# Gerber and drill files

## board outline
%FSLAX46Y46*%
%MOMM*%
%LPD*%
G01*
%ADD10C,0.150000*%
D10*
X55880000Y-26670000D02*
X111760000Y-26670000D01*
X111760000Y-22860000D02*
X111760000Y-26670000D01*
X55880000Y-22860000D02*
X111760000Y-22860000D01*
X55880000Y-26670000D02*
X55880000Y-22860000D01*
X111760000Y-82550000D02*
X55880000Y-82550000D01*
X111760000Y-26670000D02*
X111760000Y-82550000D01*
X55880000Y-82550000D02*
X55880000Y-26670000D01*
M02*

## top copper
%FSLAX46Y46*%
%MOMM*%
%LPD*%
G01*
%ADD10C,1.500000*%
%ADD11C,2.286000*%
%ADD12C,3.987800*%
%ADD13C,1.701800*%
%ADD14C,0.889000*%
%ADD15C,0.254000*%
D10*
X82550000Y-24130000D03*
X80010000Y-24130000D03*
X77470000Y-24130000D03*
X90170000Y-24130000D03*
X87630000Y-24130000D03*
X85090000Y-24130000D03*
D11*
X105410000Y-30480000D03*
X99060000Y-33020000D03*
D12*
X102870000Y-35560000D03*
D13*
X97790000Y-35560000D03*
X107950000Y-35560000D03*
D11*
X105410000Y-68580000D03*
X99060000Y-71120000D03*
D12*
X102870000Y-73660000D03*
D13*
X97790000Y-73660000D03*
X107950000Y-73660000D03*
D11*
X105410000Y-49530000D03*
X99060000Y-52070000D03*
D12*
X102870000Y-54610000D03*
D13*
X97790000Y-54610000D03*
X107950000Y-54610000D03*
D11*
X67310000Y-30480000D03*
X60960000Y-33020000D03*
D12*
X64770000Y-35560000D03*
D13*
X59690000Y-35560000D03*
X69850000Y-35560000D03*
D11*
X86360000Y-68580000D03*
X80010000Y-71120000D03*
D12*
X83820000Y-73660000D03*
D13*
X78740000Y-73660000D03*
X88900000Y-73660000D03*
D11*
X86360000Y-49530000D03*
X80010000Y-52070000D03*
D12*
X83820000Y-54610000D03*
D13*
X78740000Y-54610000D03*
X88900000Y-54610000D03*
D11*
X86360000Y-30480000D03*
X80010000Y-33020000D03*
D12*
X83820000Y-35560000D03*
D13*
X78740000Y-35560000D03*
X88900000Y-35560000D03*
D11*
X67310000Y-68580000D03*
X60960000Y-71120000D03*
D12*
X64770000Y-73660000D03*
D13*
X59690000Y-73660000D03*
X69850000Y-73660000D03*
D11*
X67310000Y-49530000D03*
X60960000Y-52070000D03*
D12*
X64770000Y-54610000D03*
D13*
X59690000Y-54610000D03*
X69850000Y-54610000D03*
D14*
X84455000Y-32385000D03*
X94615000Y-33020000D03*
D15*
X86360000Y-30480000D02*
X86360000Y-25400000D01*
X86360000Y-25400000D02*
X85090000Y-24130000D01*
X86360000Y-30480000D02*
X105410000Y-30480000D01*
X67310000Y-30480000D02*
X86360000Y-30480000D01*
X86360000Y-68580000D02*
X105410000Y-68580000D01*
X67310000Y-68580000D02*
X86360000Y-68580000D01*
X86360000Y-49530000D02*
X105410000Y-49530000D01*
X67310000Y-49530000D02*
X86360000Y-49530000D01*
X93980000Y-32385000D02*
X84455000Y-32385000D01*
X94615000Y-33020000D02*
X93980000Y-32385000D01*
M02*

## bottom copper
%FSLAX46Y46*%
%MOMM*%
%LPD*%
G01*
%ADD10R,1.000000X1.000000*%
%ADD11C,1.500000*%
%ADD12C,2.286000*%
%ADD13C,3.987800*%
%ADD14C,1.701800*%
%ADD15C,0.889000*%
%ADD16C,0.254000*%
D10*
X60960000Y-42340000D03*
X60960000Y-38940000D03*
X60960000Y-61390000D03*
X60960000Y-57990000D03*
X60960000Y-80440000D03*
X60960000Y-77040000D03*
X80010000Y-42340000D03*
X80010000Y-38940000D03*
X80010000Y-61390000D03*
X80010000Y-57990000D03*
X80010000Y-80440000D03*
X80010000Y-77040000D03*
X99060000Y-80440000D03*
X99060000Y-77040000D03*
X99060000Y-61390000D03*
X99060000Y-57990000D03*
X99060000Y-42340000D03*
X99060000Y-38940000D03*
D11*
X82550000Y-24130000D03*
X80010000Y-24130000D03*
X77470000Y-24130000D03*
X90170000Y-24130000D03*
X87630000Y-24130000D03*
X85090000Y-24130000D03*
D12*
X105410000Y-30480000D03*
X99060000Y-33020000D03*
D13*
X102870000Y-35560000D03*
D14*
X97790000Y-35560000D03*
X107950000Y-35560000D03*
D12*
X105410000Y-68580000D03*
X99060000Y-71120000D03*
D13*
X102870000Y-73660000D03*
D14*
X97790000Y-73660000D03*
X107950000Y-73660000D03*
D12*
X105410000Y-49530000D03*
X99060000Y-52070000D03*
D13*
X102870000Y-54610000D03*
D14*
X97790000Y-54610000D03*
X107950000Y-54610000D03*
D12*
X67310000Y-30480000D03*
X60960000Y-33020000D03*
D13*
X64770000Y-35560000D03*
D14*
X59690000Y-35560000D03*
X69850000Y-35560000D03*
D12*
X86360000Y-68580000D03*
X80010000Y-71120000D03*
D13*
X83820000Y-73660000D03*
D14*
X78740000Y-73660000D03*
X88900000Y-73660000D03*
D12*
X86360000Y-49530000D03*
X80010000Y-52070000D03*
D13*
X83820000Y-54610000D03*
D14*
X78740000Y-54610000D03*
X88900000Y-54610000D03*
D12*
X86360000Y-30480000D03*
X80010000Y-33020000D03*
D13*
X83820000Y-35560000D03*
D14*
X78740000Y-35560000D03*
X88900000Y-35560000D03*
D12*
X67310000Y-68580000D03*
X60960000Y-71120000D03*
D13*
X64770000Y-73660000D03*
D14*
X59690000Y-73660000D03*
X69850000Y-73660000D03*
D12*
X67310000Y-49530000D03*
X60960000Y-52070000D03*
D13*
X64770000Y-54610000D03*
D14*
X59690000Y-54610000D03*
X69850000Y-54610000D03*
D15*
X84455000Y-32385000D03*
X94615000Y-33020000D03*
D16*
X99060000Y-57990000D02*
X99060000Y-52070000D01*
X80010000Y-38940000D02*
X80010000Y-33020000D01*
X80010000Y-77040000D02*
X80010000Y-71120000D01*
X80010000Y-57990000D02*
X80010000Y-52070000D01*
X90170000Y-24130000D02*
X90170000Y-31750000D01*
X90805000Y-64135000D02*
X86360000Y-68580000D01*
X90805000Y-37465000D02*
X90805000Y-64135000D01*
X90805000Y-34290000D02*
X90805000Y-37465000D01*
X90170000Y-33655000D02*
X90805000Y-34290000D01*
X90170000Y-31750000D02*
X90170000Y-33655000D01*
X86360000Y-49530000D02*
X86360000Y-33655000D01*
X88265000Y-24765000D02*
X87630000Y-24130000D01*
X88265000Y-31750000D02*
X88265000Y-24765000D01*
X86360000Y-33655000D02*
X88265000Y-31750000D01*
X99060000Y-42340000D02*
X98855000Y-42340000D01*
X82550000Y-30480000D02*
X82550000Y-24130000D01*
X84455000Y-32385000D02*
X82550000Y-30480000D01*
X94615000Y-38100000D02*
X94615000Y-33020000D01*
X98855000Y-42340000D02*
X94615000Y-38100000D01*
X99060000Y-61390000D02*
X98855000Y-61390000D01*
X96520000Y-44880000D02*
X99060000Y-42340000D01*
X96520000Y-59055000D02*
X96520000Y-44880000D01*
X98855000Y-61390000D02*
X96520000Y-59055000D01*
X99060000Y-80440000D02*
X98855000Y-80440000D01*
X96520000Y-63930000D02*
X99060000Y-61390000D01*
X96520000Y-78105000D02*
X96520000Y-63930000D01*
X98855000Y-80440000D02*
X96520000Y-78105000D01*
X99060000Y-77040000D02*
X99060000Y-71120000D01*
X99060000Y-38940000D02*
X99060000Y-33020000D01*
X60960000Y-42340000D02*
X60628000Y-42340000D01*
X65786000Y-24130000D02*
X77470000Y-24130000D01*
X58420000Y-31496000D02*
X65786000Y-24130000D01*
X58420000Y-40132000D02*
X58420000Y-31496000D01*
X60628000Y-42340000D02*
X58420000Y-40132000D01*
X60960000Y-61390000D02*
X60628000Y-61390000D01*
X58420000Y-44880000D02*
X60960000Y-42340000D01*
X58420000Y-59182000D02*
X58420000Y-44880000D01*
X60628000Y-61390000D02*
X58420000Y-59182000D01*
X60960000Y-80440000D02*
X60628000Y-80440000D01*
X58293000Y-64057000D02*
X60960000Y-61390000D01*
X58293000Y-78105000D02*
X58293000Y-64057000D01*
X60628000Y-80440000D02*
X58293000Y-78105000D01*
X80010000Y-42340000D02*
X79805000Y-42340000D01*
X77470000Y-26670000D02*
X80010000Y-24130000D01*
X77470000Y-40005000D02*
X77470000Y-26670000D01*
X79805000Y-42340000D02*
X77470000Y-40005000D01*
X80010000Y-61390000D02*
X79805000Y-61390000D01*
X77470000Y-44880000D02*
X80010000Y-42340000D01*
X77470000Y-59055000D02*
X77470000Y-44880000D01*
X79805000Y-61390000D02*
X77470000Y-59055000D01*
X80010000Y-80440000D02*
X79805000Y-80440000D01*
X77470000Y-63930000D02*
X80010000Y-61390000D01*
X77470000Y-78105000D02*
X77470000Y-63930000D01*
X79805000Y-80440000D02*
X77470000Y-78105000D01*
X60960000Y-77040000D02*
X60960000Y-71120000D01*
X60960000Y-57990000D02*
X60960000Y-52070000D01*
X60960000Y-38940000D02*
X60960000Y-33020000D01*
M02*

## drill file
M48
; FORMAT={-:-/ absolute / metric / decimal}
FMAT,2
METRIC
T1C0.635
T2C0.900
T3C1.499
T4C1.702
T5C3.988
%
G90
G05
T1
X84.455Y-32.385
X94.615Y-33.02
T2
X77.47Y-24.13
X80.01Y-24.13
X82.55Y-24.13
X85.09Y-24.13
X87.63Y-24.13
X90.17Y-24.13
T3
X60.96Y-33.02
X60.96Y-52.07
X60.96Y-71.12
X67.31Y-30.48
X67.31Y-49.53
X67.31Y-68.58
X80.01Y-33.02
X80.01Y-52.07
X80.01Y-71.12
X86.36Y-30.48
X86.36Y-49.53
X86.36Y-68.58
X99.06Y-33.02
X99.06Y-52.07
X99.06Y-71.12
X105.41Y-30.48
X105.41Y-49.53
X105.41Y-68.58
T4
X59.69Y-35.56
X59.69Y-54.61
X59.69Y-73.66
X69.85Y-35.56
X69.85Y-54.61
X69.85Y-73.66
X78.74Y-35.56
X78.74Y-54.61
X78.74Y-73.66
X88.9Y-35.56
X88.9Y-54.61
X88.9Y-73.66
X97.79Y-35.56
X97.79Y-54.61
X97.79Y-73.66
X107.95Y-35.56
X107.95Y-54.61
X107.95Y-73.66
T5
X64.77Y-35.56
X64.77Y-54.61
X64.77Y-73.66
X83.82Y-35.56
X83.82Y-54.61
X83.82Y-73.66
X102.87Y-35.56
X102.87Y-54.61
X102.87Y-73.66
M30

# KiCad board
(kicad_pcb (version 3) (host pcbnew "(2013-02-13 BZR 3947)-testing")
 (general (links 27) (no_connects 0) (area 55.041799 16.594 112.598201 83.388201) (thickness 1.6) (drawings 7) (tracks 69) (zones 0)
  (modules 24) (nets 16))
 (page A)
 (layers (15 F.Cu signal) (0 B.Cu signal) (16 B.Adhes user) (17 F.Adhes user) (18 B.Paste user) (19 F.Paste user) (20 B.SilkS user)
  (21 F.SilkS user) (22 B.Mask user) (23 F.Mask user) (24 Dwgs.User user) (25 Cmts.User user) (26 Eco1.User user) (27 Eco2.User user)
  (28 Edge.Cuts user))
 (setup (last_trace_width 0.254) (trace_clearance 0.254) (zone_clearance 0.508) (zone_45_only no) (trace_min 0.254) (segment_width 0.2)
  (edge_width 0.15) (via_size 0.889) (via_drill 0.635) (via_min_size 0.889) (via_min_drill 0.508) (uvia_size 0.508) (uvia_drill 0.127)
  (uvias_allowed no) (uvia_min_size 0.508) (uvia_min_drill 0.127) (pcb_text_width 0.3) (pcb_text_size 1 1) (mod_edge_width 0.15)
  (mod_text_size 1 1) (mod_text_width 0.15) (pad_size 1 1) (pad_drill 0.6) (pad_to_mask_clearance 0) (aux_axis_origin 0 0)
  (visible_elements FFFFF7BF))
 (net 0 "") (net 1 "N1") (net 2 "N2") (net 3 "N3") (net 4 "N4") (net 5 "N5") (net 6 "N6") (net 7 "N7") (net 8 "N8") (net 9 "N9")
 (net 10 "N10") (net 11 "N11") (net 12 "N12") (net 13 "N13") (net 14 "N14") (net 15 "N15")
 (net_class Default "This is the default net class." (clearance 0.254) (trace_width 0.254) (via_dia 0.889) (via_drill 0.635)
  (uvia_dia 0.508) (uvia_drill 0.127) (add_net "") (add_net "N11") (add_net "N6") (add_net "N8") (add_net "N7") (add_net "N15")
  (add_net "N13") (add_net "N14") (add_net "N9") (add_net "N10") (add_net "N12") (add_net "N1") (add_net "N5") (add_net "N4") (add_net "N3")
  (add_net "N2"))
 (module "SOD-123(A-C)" (layer B.Cu) (at 60.96 40.64 90)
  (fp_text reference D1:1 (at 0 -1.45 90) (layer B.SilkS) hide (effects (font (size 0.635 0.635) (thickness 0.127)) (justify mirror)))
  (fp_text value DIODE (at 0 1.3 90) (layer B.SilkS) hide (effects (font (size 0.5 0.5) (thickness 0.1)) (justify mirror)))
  (pad A smd rect (at -1.7 0 90) (size 1 1) (layers B.Cu B.Paste B.Mask) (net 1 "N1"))
  (pad C smd rect (at 1.7 0 90) (size 1 1) (layers B.Cu B.Paste B.Mask) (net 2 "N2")))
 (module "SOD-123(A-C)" (layer B.Cu) (at 60.96 59.69 90)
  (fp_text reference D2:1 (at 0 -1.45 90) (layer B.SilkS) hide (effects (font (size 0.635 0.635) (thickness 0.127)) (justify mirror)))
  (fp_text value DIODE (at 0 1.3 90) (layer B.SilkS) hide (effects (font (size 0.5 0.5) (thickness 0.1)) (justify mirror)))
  (pad A smd rect (at -1.7 0 90) (size 1 1) (layers B.Cu B.Paste B.Mask) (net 1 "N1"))
  (pad C smd rect (at 1.7 0 90) (size 1 1) (layers B.Cu B.Paste B.Mask) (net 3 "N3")))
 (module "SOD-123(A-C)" (layer B.Cu) (at 60.96 78.74 90)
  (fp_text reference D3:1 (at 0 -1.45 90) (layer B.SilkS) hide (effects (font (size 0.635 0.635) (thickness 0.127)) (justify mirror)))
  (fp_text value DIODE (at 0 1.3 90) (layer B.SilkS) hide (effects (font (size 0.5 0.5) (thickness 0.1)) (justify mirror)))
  (pad A smd rect (at -1.7 0 90) (size 1 1) (layers B.Cu B.Paste B.Mask) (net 1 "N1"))
  (pad C smd rect (at 1.7 0 90) (size 1 1) (layers B.Cu B.Paste B.Mask) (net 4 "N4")))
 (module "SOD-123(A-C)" (layer B.Cu) (at 80.01 40.64 90)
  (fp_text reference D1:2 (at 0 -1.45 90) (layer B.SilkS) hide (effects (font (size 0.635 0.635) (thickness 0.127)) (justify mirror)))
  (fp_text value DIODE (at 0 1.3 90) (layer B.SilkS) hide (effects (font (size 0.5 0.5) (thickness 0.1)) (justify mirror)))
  (pad A smd rect (at -1.7 0 90) (size 1 1) (layers B.Cu B.Paste B.Mask) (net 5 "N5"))
  (pad C smd rect (at 1.7 0 90) (size 1 1) (layers B.Cu B.Paste B.Mask) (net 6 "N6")))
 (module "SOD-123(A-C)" (layer B.Cu) (at 80.01 59.69 90)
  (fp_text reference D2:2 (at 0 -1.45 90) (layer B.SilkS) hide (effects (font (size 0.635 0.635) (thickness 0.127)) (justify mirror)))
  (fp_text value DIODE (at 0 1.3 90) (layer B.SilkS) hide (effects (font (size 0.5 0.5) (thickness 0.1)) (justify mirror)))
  (pad A smd rect (at -1.7 0 90) (size 1 1) (layers B.Cu B.Paste B.Mask) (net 5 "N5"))
  (pad C smd rect (at 1.7 0 90) (size 1 1) (layers B.Cu B.Paste B.Mask) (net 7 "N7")))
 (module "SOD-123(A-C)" (layer B.Cu) (at 80.01 78.74 90)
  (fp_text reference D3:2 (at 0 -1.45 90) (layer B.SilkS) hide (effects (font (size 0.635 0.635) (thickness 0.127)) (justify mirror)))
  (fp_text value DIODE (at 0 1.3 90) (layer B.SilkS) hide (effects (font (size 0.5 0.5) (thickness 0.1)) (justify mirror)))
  (pad A smd rect (at -1.7 0 90) (size 1 1) (layers B.Cu B.Paste B.Mask) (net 5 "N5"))
  (pad C smd rect (at 1.7 0 90) (size 1 1) (layers B.Cu B.Paste B.Mask) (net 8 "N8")))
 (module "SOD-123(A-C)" (layer B.Cu) (at 99.06 78.74 90)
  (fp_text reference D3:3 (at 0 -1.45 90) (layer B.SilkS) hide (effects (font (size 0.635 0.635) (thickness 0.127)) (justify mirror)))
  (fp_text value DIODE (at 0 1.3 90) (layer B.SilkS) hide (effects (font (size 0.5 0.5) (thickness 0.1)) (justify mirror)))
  (pad A smd rect (at -1.7 0 90) (size 1 1) (layers B.Cu B.Paste B.Mask) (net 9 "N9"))
  (pad C smd rect (at 1.7 0 90) (size 1 1) (layers B.Cu B.Paste B.Mask) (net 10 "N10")))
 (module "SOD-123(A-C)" (layer B.Cu) (at 99.06 59.69 90)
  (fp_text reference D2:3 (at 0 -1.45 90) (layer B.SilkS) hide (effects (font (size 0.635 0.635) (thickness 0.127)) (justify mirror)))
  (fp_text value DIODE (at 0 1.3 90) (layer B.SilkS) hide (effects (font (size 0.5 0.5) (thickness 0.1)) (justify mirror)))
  (pad A smd rect (at -1.7 0 90) (size 1 1) (layers B.Cu B.Paste B.Mask) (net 9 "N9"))
  (pad C smd rect (at 1.7 0 90) (size 1 1) (layers B.Cu B.Paste B.Mask) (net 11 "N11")))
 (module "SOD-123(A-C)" (layer B.Cu) (at 99.06 40.64 90)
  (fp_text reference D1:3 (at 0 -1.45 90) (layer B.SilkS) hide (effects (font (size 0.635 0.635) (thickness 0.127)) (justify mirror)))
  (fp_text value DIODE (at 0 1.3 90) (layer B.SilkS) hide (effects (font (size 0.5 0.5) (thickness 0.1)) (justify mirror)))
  (pad A smd rect (at -1.7 0 90) (size 1 1) (layers B.Cu B.Paste B.Mask) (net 9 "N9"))
  (pad C smd rect (at 1.7 0 90) (size 1 1) (layers B.Cu B.Paste B.Mask) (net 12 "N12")))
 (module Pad (layer F.Cu) (at 82.55 24.13)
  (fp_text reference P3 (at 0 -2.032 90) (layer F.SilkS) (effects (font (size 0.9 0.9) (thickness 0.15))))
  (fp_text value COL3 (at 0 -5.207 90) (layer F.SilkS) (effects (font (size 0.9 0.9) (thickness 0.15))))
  (pad 1 thru_hole circle (at 0 0) (size 1.5 1.5) (drill 0.9) (layers *.Cu *.Mask F.SilkS) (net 9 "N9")))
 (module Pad (layer F.Cu) (at 80.01 24.13)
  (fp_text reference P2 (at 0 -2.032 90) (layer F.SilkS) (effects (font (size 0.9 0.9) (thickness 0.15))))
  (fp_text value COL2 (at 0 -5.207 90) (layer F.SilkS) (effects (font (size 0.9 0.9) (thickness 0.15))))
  (pad 1 thru_hole circle (at 0 0) (size 1.5 1.5) (drill 0.9) (layers *.Cu *.Mask F.SilkS) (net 5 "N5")))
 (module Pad (layer F.Cu) (at 77.47 24.13)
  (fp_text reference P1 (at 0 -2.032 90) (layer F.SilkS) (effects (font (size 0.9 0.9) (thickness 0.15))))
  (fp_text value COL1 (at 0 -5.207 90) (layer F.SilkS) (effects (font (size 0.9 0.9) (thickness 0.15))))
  (pad 1 thru_hole circle (at 0 0) (size 1.5 1.5) (drill 0.9) (layers *.Cu *.Mask F.SilkS) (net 1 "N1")))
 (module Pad (layer F.Cu) (at 90.17 24.13)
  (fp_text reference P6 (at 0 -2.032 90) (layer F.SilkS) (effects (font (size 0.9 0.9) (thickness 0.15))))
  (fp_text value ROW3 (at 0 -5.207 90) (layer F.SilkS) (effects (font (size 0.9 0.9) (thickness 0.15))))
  (pad 1 thru_hole circle (at 0 0) (size 1.5 1.5) (drill 0.9) (layers *.Cu *.Mask F.SilkS) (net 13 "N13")))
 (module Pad (layer F.Cu) (at 87.63 24.13)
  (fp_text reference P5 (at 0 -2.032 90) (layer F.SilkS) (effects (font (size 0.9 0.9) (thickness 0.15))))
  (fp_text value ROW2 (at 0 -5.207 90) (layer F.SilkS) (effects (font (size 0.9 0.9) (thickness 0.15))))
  (pad 1 thru_hole circle (at 0 0) (size 1.5 1.5) (drill 0.9) (layers *.Cu *.Mask F.SilkS) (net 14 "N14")))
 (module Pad (layer F.Cu) (at 85.09 24.13)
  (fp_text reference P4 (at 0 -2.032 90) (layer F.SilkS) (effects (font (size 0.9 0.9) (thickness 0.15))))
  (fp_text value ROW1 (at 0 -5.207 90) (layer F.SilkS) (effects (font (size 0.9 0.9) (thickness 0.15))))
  (pad 1 thru_hole circle (at 0 0) (size 1.5 1.5) (drill 0.9) (layers *.Cu *.Mask F.SilkS) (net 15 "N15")))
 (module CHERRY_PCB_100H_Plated (layer F.Cu) (at 102.87 35.56)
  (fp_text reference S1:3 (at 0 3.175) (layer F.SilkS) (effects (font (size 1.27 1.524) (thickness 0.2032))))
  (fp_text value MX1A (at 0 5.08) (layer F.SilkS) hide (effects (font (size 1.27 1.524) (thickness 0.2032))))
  (pad 1 thru_hole circle (at 2.54 -5.08) (size 2.286 2.286) (drill 1.4986) (layers *.Cu *.SilkS *.Mask) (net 15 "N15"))
  (pad 2 thru_hole circle (at -3.81 -2.54) (size 2.286 2.286) (drill 1.4986) (layers *.Cu *.SilkS *.Mask) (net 12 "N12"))
  (pad HOLE thru_hole circle (at 0 0) (size 3.9878 3.9878) (drill 3.9878) (layers *.Cu *.Mask F.SilkS))
  (pad HOLE thru_hole circle (at -5.08 0) (size 1.7018 1.7018) (drill 1.7018) (layers *.Cu *.Mask F.SilkS))
  (pad HOLE thru_hole circle (at 5.08 0) (size 1.7018 1.7018) (drill 1.7018) (layers *.Cu *.Mask F.SilkS)))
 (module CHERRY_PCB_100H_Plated (layer F.Cu) (at 102.87 73.66)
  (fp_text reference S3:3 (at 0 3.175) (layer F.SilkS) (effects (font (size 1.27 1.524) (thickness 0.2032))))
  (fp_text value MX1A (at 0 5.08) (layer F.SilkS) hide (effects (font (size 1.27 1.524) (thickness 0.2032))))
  (pad 1 thru_hole circle (at 2.54 -5.08) (size 2.286 2.286) (drill 1.4986) (layers *.Cu *.SilkS *.Mask) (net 13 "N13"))
  (pad 2 thru_hole circle (at -3.81 -2.54) (size 2.286 2.286) (drill 1.4986) (layers *.Cu *.SilkS *.Mask) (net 10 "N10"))
  (pad HOLE thru_hole circle (at 0 0) (size 3.9878 3.9878) (drill 3.9878) (layers *.Cu *.Mask F.SilkS))
  (pad HOLE thru_hole circle (at -5.08 0) (size 1.7018 1.7018) (drill 1.7018) (layers *.Cu *.Mask F.SilkS))
  (pad HOLE thru_hole circle (at 5.08 0) (size 1.7018 1.7018) (drill 1.7018) (layers *.Cu *.Mask F.SilkS)))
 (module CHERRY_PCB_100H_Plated (layer F.Cu) (at 102.87 54.61)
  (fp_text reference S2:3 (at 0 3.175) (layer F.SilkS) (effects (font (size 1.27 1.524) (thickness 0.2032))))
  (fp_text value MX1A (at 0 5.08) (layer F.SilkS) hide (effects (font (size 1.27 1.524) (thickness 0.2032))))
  (pad 1 thru_hole circle (at 2.54 -5.08) (size 2.286 2.286) (drill 1.4986) (layers *.Cu *.SilkS *.Mask) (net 14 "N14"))
  (pad 2 thru_hole circle (at -3.81 -2.54) (size 2.286 2.286) (drill 1.4986) (layers *.Cu *.SilkS *.Mask) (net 11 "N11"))
  (pad HOLE thru_hole circle (at 0 0) (size 3.9878 3.9878) (drill 3.9878) (layers *.Cu *.Mask F.SilkS))
  (pad HOLE thru_hole circle (at -5.08 0) (size 1.7018 1.7018) (drill 1.7018) (layers *.Cu *.Mask F.SilkS))
  (pad HOLE thru_hole circle (at 5.08 0) (size 1.7018 1.7018) (drill 1.7018) (layers *.Cu *.Mask F.SilkS)))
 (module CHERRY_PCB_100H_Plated (layer F.Cu) (at 64.77 35.56)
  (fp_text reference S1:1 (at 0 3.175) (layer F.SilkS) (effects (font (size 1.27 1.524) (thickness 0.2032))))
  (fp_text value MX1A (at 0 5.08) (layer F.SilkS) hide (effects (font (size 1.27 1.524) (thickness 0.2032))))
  (pad 1 thru_hole circle (at 2.54 -5.08) (size 2.286 2.286) (drill 1.4986) (layers *.Cu *.SilkS *.Mask) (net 15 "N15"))
  (pad 2 thru_hole circle (at -3.81 -2.54) (size 2.286 2.286) (drill 1.4986) (layers *.Cu *.SilkS *.Mask) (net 2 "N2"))
  (pad HOLE thru_hole circle (at 0 0) (size 3.9878 3.9878) (drill 3.9878) (layers *.Cu *.Mask F.SilkS))
  (pad HOLE thru_hole circle (at -5.08 0) (size 1.7018 1.7018) (drill 1.7018) (layers *.Cu *.Mask F.SilkS))
  (pad HOLE thru_hole circle (at 5.08 0) (size 1.7018 1.7018) (drill 1.7018) (layers *.Cu *.Mask F.SilkS)))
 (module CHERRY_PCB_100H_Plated (layer F.Cu) (at 83.82 73.66)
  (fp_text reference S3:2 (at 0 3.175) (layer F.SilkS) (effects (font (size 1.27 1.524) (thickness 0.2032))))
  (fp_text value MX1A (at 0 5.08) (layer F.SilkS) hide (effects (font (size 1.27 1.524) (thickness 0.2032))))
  (pad 1 thru_hole circle (at 2.54 -5.08) (size 2.286 2.286) (drill 1.4986) (layers *.Cu *.SilkS *.Mask) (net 13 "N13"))
  (pad 2 thru_hole circle (at -3.81 -2.54) (size 2.286 2.286) (drill 1.4986) (layers *.Cu *.SilkS *.Mask) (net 8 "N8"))
  (pad HOLE thru_hole circle (at 0 0) (size 3.9878 3.9878) (drill 3.9878) (layers *.Cu *.Mask F.SilkS))
  (pad HOLE thru_hole circle (at -5.08 0) (size 1.7018 1.7018) (drill 1.7018) (layers *.Cu *.Mask F.SilkS))
  (pad HOLE thru_hole circle (at 5.08 0) (size 1.7018 1.7018) (drill 1.7018) (layers *.Cu *.Mask F.SilkS)))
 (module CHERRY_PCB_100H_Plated (layer F.Cu) (at 83.82 54.61)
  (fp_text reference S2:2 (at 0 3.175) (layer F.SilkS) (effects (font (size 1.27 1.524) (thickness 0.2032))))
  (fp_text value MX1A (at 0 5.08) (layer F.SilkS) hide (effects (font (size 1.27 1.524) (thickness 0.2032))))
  (pad 1 thru_hole circle (at 2.54 -5.08) (size 2.286 2.286) (drill 1.4986) (layers *.Cu *.SilkS *.Mask) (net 14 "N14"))
  (pad 2 thru_hole circle (at -3.81 -2.54) (size 2.286 2.286) (drill 1.4986) (layers *.Cu *.SilkS *.Mask) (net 7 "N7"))
  (pad HOLE thru_hole circle (at 0 0) (size 3.9878 3.9878) (drill 3.9878) (layers *.Cu *.Mask F.SilkS))
  (pad HOLE thru_hole circle (at -5.08 0) (size 1.7018 1.7018) (drill 1.7018) (layers *.Cu *.Mask F.SilkS))
  (pad HOLE thru_hole circle (at 5.08 0) (size 1.7018 1.7018) (drill 1.7018) (layers *.Cu *.Mask F.SilkS)))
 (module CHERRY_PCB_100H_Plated (layer F.Cu) (at 83.82 35.56)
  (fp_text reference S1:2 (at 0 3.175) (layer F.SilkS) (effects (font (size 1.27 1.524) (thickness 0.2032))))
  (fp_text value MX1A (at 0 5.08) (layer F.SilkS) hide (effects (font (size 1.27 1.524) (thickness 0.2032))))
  (pad 1 thru_hole circle (at 2.54 -5.08) (size 2.286 2.286) (drill 1.4986) (layers *.Cu *.SilkS *.Mask) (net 15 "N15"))
  (pad 2 thru_hole circle (at -3.81 -2.54) (size 2.286 2.286) (drill 1.4986) (layers *.Cu *.SilkS *.Mask) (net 6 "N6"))
  (pad HOLE thru_hole circle (at 0 0) (size 3.9878 3.9878) (drill 3.9878) (layers *.Cu *.Mask F.SilkS))
  (pad HOLE thru_hole circle (at -5.08 0) (size 1.7018 1.7018) (drill 1.7018) (layers *.Cu *.Mask F.SilkS))
  (pad HOLE thru_hole circle (at 5.08 0) (size 1.7018 1.7018) (drill 1.7018) (layers *.Cu *.Mask F.SilkS)))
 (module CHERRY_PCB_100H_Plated (layer F.Cu) (at 64.77 73.66)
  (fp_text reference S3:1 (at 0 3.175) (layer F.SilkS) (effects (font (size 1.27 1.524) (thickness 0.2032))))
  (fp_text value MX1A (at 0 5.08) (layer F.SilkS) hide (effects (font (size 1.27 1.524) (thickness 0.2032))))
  (pad 1 thru_hole circle (at 2.54 -5.08) (size 2.286 2.286) (drill 1.4986) (layers *.Cu *.SilkS *.Mask) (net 13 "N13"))
  (pad 2 thru_hole circle (at -3.81 -2.54) (size 2.286 2.286) (drill 1.4986) (layers *.Cu *.SilkS *.Mask) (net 4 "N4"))
  (pad HOLE thru_hole circle (at 0 0) (size 3.9878 3.9878) (drill 3.9878) (layers *.Cu *.Mask F.SilkS))
  (pad HOLE thru_hole circle (at -5.08 0) (size 1.7018 1.7018) (drill 1.7018) (layers *.Cu *.Mask F.SilkS))
  (pad HOLE thru_hole circle (at 5.08 0) (size 1.7018 1.7018) (drill 1.7018) (layers *.Cu *.Mask F.SilkS)))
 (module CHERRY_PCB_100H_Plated (layer F.Cu) (at 64.77 54.61)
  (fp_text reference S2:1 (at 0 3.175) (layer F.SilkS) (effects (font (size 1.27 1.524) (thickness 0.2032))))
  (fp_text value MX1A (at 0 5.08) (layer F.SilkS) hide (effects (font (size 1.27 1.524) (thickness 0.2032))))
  (pad 1 thru_hole circle (at 2.54 -5.08) (size 2.286 2.286) (drill 1.4986) (layers *.Cu *.SilkS *.Mask) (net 14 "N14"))
  (pad 2 thru_hole circle (at -3.81 -2.54) (size 2.286 2.286) (drill 1.4986) (layers *.Cu *.SilkS *.Mask) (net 3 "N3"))
  (pad HOLE thru_hole circle (at 0 0) (size 3.9878 3.9878) (drill 3.9878) (layers *.Cu *.Mask F.SilkS))
  (pad HOLE thru_hole circle (at -5.08 0) (size 1.7018 1.7018) (drill 1.7018) (layers *.Cu *.Mask F.SilkS))
  (pad HOLE thru_hole circle (at 5.08 0) (size 1.7018 1.7018) (drill 1.7018) (layers *.Cu *.Mask F.SilkS)))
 (gr_line (start 55.88 26.67) (end 111.76 26.67) (angle 90) (layer Edge.Cuts) (width 0.15))
 (gr_line (start 111.76 22.86) (end 111.76 26.67) (angle 90) (layer Edge.Cuts) (width 0.15))
 (gr_line (start 55.88 22.86) (end 111.76 22.86) (angle 90) (layer Edge.Cuts) (width 0.15))
 (gr_line (start 55.88 26.67) (end 55.88 22.86) (angle 90) (layer Edge.Cuts) (width 0.15))
 (gr_line (start 111.76 82.55) (end 55.88 82.55) (angle 90) (layer Edge.Cuts) (width 0.15))
 (gr_line (start 111.76 26.67) (end 111.76 82.55) (angle 90) (layer Edge.Cuts) (width 0.15))
 (gr_line (start 55.88 82.55) (end 55.88 26.67) (angle 90) (layer Edge.Cuts) (width 0.15))
 (segment (start 99.06 57.99) (end 99.06 52.07) (width 0.254) (layer B.Cu) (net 11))
 (segment (start 80.01 38.94) (end 80.01 33.02) (width 0.254) (layer B.Cu) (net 6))
 (segment (start 80.01 77.04) (end 80.01 71.12) (width 0.254) (layer B.Cu) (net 8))
 (segment (start 80.01 57.99) (end 80.01 52.07) (width 0.254) (layer B.Cu) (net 7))
 (segment (start 86.36 30.48) (end 86.36 25.4) (width 0.254) (layer F.Cu) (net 15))
 (segment (start 86.36 25.4) (end 85.09 24.13) (width 0.254) (layer F.Cu) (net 15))
 (segment (start 86.36 30.48) (end 105.41 30.48) (width 0.254) (layer F.Cu) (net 15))
 (segment (start 67.31 30.48) (end 86.36 30.48) (width 0.254) (layer F.Cu) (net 15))
 (segment (start 90.17 24.13) (end 90.17 31.75) (width 0.254) (layer B.Cu) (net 13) (status 400000))
 (segment (start 90.805 64.135) (end 86.36 68.58) (width 0.254) (layer B.Cu) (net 13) (status 800000))
 (segment (start 90.805 37.465) (end 90.805 64.135) (width 0.254) (layer B.Cu) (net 13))
 (segment (start 90.805 34.29) (end 90.805 37.465) (width 0.254) (layer B.Cu) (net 13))
 (segment (start 90.17 33.655) (end 90.805 34.29) (width 0.254) (layer B.Cu) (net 13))
 (segment (start 90.17 31.75) (end 90.17 33.655) (width 0.254) (layer B.Cu) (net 13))
 (segment (start 86.36 68.58) (end 105.41 68.58) (width 0.254) (layer F.Cu) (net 13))
 (segment (start 67.31 68.58) (end 86.36 68.58) (width 0.254) (layer F.Cu) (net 13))
 (segment (start 86.36 49.53) (end 86.36 33.655) (width 0.254) (layer B.Cu) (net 14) (status 400000))
 (segment (start 88.265 24.765) (end 87.63 24.13) (width 0.254) (layer B.Cu) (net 14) (status 800000))
 (segment (start 88.265 31.75) (end 88.265 24.765) (width 0.254) (layer B.Cu) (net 14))
 (segment (start 86.36 33.655) (end 88.265 31.75) (width 0.254) (layer B.Cu) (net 14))
 (segment (start 86.36 49.53) (end 105.41 49.53) (width 0.254) (layer F.Cu) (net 14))
 (segment (start 67.31 49.53) (end 86.36 49.53) (width 0.254) (layer F.Cu) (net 14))
 (segment (start 99.06 42.34) (end 98.855 42.34) (width 0.254) (layer B.Cu) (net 9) (status C00000))
 (segment (start 82.55 30.48) (end 82.55 24.13) (width 0.254) (layer B.Cu) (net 9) (status 800000))
 (segment (start 84.455 32.385) (end 82.55 30.48) (width 0.254) (layer B.Cu) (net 9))
 (via (at 84.455 32.385) (size 0.889) (layers F.Cu B.Cu) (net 9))
 (segment (start 93.98 32.385) (end 84.455 32.385) (width 0.254) (layer F.Cu) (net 9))
 (segment (start 94.615 33.02) (end 93.98 32.385) (width 0.254) (layer F.Cu) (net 9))
 (via (at 94.615 33.02) (size 0.889) (layers F.Cu B.Cu) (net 9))
 (segment (start 94.615 38.1) (end 94.615 33.02) (width 0.254) (layer B.Cu) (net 9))
 (segment (start 98.855 42.34) (end 94.615 38.1) (width 0.254) (layer B.Cu) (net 9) (status 400000))
 (segment (start 99.06 61.39) (end 98.855 61.39) (width 0.254) (layer B.Cu) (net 9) (status C00000))
 (segment (start 96.52 44.88) (end 99.06 42.34) (width 0.254) (layer B.Cu) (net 9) (status 800000))
 (segment (start 96.52 59.055) (end 96.52 44.88) (width 0.254) (layer B.Cu) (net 9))
 (segment (start 98.855 61.39) (end 96.52 59.055) (width 0.254) (layer B.Cu) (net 9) (status 400000))
 (segment (start 99.06 80.44) (end 98.855 80.44) (width 0.254) (layer B.Cu) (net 9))
 (segment (start 96.52 63.93) (end 99.06 61.39) (width 0.254) (layer B.Cu) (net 9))
 (segment (start 96.52 78.105) (end 96.52 63.93) (width 0.254) (layer B.Cu) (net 9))
 (segment (start 98.855 80.44) (end 96.52 78.105) (width 0.254) (layer B.Cu) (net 9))
 (segment (start 99.06 77.04) (end 99.06 71.12) (width 0.254) (layer B.Cu) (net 10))
 (segment (start 99.06 38.94) (end 99.06 33.02) (width 0.254) (layer B.Cu) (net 12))
 (segment (start 60.96 42.34) (end 60.628 42.34) (width 0.254) (layer B.Cu) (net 1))
 (segment (start 65.786 24.13) (end 77.47 24.13) (width 0.254) (layer B.Cu) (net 1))
 (segment (start 58.42 31.496) (end 65.786 24.13) (width 0.254) (layer B.Cu) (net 1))
 (segment (start 58.42 40.132) (end 58.42 31.496) (width 0.254) (layer B.Cu) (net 1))
 (segment (start 60.628 42.34) (end 58.42 40.132) (width 0.254) (layer B.Cu) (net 1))
 (segment (start 60.96 61.39) (end 60.628 61.39) (width 0.254) (layer B.Cu) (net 1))
 (segment (start 58.42 44.88) (end 60.96 42.34) (width 0.254) (layer B.Cu) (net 1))
 (segment (start 58.42 59.182) (end 58.42 44.88) (width 0.254) (layer B.Cu) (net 1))
 (segment (start 60.628 61.39) (end 58.42 59.182) (width 0.254) (layer B.Cu) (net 1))
 (segment (start 60.96 80.44) (end 60.628 80.44) (width 0.254) (layer B.Cu) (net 1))
 (segment (start 58.293 64.057) (end 60.96 61.39) (width 0.254) (layer B.Cu) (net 1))
 (segment (start 58.293 78.105) (end 58.293 64.057) (width 0.254) (layer B.Cu) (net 1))
 (segment (start 60.628 80.44) (end 58.293 78.105) (width 0.254) (layer B.Cu) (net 1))
 (segment (start 80.01 42.34) (end 79.805 42.34) (width 0.254) (layer B.Cu) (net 5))
 (segment (start 77.47 26.67) (end 80.01 24.13) (width 0.254) (layer B.Cu) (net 5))
 (segment (start 77.47 40.005) (end 77.47 26.67) (width 0.254) (layer B.Cu) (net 5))
 (segment (start 79.805 42.34) (end 77.47 40.005) (width 0.254) (layer B.Cu) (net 5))
 (segment (start 80.01 61.39) (end 79.805 61.39) (width 0.254) (layer B.Cu) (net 5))
 (segment (start 77.47 44.88) (end 80.01 42.34) (width 0.254) (layer B.Cu) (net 5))
 (segment (start 77.47 59.055) (end 77.47 44.88) (width 0.254) (layer B.Cu) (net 5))
 (segment (start 79.805 61.39) (end 77.47 59.055) (width 0.254) (layer B.Cu) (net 5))
 (segment (start 80.01 80.44) (end 79.805 80.44) (width 0.254) (layer B.Cu) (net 5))
 (segment (start 77.47 63.93) (end 80.01 61.39) (width 0.254) (layer B.Cu) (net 5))
 (segment (start 77.47 78.105) (end 77.47 63.93) (width 0.254) (layer B.Cu) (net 5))
 (segment (start 79.805 80.44) (end 77.47 78.105) (width 0.254) (layer B.Cu) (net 5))
 (segment (start 60.96 77.04) (end 60.96 71.12) (width 0.254) (layer B.Cu) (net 4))
 (segment (start 60.96 57.99) (end 60.96 52.07) (width 0.254) (layer B.Cu) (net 3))
 (segment (start 60.96 38.94) (end 60.96 33.02) (width 0.254) (layer B.Cu) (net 2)))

